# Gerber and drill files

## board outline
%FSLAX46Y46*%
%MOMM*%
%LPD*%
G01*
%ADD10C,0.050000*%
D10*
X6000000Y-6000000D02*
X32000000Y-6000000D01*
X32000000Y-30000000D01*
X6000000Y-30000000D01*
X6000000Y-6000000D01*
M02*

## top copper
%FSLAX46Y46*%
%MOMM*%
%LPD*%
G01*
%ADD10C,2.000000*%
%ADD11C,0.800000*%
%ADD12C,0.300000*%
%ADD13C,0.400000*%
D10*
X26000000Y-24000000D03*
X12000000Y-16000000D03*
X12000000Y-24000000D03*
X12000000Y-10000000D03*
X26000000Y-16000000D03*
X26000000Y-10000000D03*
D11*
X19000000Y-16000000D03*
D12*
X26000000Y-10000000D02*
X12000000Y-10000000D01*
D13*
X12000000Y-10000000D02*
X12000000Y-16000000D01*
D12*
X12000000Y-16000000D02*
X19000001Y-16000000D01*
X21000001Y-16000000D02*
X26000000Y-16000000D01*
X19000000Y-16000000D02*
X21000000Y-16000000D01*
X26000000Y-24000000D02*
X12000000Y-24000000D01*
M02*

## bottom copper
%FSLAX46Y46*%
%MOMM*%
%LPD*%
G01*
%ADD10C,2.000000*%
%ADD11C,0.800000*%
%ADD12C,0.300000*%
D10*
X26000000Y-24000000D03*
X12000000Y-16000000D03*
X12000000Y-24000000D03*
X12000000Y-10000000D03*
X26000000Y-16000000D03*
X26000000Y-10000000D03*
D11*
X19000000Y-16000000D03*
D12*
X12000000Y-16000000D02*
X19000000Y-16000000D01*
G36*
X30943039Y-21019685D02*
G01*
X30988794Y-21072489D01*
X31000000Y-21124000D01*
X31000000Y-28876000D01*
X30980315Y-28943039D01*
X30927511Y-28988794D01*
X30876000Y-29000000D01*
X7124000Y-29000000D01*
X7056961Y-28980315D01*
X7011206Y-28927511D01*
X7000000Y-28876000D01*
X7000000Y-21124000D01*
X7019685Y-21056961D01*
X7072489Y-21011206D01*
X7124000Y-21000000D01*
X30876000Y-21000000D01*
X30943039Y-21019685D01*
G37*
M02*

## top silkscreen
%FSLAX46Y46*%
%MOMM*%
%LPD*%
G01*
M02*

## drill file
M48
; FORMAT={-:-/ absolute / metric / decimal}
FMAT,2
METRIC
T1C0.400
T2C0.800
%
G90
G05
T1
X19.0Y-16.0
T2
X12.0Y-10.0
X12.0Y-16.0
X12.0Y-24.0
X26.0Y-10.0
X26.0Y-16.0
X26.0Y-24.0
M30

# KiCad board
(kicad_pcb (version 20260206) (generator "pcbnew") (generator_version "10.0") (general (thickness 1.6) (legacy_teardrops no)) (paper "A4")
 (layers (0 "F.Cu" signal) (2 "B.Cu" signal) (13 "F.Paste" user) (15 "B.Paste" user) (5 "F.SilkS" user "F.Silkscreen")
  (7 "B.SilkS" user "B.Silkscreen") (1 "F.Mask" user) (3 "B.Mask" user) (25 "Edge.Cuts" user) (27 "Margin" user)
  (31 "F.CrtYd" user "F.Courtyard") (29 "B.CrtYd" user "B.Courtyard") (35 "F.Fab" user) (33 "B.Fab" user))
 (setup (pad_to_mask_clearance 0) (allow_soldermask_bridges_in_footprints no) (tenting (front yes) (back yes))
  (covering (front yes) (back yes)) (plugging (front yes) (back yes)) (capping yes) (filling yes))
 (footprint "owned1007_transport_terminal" (layer "F.Cu") (at 26 24)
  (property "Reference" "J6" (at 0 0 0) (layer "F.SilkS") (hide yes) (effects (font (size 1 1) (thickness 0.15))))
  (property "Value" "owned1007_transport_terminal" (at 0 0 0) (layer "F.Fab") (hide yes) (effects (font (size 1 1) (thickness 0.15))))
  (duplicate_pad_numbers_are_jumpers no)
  (pad "1" thru_hole circle (at 0 0) (size 2 2) (drill 0.8) (layers "*.Cu" "*.Mask") (remove_unused_layers no) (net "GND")))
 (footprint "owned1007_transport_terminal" (layer "F.Cu") (at 12 16)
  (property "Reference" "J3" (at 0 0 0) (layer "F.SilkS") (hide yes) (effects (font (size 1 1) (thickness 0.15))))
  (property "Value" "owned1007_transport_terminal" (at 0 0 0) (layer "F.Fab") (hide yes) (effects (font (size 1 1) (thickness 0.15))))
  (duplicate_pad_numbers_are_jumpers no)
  (pad "1" thru_hole circle (at 0 0) (size 2 2) (drill 0.8) (layers "*.Cu" "*.Mask") (remove_unused_layers no) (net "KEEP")))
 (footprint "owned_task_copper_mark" (layer "F.Cu") (at 10 28)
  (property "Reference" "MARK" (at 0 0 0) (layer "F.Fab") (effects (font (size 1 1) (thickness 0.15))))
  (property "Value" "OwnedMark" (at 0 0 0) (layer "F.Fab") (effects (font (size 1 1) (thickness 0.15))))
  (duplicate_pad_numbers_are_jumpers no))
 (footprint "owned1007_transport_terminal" (layer "F.Cu") (at 12 24)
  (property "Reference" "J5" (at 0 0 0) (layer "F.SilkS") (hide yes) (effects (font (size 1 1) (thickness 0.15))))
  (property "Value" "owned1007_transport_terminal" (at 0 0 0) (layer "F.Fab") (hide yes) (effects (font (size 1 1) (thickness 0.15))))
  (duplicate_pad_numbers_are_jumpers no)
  (pad "1" thru_hole circle (at 0 0) (size 2 2) (drill 0.8) (layers "*.Cu" "*.Mask") (remove_unused_layers no) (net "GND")))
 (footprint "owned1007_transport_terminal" (layer "F.Cu") (at 12 10)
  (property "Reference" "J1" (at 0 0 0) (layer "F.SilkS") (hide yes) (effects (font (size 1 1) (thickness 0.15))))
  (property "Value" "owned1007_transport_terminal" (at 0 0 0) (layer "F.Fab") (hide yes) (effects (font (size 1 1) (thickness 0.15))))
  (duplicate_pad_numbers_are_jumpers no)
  (pad "1" thru_hole circle (at 0 0) (size 2 2) (drill 0.8) (layers "*.Cu" "*.Mask") (remove_unused_layers no) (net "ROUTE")))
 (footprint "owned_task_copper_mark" (layer "F.Cu") (at 13 28)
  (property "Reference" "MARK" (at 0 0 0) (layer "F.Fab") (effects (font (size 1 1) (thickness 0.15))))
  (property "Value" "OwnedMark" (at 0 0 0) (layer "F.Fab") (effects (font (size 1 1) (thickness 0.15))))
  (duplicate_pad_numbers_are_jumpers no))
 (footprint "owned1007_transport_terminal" (layer "F.Cu") (at 26 16)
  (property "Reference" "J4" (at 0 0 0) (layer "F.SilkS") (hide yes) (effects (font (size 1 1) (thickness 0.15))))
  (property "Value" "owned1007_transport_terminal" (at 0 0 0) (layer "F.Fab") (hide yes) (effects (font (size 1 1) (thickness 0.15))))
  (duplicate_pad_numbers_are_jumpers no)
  (pad "1" thru_hole circle (at 0 0) (size 2 2) (drill 0.8) (layers "*.Cu" "*.Mask") (remove_unused_layers no) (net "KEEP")))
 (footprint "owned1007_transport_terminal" (layer "F.Cu") (at 26 10)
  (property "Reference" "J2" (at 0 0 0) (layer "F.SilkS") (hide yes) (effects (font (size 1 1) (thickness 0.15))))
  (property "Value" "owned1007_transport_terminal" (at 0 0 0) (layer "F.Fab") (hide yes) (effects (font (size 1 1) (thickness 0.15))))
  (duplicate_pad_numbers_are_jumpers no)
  (pad "1" thru_hole circle (at 0 0) (size 2 2) (drill 0.8) (layers "*.Cu" "*.Mask") (remove_unused_layers no) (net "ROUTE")))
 (gr_rect (start 6 6) (end 32 30) (stroke (width 0.05) (type default)) (fill no) (layer "Edge.Cuts"))
 (segment (start 26 10) (end 12 10) (width 0.3) (layer "F.Cu") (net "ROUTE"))
 (segment (start 12 10) (end 12 16) (width 0.4) (layer "F.Cu") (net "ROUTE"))
 (segment (start 12 16) (end 19.000001 16) (width 0.3) (layer "F.Cu") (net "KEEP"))
 (segment (start 21.000001 16) (end 26 16) (width 0.3) (layer "F.Cu") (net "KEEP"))
 (segment (start 19 16) (end 21 16) (width 0.3) (layer "F.Cu") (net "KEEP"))
 (via (at 19 16) (size 0.8) (drill 0.4) (layers "F.Cu" "B.Cu") (free yes) (capping no) (covering (front no) (back no))
  (plugging (front no) (back no)) (filling no) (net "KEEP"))
 (segment (start 12 16) (end 19 16) (width 0.3) (locked yes) (layer "B.Cu") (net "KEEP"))
 (segment (start 26 24) (end 12 24) (width 0.3) (layer "F.Cu") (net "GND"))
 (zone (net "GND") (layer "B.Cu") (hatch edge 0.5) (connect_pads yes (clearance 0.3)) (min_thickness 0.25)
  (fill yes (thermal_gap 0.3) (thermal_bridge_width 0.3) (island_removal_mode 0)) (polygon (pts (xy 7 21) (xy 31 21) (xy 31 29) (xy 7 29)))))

